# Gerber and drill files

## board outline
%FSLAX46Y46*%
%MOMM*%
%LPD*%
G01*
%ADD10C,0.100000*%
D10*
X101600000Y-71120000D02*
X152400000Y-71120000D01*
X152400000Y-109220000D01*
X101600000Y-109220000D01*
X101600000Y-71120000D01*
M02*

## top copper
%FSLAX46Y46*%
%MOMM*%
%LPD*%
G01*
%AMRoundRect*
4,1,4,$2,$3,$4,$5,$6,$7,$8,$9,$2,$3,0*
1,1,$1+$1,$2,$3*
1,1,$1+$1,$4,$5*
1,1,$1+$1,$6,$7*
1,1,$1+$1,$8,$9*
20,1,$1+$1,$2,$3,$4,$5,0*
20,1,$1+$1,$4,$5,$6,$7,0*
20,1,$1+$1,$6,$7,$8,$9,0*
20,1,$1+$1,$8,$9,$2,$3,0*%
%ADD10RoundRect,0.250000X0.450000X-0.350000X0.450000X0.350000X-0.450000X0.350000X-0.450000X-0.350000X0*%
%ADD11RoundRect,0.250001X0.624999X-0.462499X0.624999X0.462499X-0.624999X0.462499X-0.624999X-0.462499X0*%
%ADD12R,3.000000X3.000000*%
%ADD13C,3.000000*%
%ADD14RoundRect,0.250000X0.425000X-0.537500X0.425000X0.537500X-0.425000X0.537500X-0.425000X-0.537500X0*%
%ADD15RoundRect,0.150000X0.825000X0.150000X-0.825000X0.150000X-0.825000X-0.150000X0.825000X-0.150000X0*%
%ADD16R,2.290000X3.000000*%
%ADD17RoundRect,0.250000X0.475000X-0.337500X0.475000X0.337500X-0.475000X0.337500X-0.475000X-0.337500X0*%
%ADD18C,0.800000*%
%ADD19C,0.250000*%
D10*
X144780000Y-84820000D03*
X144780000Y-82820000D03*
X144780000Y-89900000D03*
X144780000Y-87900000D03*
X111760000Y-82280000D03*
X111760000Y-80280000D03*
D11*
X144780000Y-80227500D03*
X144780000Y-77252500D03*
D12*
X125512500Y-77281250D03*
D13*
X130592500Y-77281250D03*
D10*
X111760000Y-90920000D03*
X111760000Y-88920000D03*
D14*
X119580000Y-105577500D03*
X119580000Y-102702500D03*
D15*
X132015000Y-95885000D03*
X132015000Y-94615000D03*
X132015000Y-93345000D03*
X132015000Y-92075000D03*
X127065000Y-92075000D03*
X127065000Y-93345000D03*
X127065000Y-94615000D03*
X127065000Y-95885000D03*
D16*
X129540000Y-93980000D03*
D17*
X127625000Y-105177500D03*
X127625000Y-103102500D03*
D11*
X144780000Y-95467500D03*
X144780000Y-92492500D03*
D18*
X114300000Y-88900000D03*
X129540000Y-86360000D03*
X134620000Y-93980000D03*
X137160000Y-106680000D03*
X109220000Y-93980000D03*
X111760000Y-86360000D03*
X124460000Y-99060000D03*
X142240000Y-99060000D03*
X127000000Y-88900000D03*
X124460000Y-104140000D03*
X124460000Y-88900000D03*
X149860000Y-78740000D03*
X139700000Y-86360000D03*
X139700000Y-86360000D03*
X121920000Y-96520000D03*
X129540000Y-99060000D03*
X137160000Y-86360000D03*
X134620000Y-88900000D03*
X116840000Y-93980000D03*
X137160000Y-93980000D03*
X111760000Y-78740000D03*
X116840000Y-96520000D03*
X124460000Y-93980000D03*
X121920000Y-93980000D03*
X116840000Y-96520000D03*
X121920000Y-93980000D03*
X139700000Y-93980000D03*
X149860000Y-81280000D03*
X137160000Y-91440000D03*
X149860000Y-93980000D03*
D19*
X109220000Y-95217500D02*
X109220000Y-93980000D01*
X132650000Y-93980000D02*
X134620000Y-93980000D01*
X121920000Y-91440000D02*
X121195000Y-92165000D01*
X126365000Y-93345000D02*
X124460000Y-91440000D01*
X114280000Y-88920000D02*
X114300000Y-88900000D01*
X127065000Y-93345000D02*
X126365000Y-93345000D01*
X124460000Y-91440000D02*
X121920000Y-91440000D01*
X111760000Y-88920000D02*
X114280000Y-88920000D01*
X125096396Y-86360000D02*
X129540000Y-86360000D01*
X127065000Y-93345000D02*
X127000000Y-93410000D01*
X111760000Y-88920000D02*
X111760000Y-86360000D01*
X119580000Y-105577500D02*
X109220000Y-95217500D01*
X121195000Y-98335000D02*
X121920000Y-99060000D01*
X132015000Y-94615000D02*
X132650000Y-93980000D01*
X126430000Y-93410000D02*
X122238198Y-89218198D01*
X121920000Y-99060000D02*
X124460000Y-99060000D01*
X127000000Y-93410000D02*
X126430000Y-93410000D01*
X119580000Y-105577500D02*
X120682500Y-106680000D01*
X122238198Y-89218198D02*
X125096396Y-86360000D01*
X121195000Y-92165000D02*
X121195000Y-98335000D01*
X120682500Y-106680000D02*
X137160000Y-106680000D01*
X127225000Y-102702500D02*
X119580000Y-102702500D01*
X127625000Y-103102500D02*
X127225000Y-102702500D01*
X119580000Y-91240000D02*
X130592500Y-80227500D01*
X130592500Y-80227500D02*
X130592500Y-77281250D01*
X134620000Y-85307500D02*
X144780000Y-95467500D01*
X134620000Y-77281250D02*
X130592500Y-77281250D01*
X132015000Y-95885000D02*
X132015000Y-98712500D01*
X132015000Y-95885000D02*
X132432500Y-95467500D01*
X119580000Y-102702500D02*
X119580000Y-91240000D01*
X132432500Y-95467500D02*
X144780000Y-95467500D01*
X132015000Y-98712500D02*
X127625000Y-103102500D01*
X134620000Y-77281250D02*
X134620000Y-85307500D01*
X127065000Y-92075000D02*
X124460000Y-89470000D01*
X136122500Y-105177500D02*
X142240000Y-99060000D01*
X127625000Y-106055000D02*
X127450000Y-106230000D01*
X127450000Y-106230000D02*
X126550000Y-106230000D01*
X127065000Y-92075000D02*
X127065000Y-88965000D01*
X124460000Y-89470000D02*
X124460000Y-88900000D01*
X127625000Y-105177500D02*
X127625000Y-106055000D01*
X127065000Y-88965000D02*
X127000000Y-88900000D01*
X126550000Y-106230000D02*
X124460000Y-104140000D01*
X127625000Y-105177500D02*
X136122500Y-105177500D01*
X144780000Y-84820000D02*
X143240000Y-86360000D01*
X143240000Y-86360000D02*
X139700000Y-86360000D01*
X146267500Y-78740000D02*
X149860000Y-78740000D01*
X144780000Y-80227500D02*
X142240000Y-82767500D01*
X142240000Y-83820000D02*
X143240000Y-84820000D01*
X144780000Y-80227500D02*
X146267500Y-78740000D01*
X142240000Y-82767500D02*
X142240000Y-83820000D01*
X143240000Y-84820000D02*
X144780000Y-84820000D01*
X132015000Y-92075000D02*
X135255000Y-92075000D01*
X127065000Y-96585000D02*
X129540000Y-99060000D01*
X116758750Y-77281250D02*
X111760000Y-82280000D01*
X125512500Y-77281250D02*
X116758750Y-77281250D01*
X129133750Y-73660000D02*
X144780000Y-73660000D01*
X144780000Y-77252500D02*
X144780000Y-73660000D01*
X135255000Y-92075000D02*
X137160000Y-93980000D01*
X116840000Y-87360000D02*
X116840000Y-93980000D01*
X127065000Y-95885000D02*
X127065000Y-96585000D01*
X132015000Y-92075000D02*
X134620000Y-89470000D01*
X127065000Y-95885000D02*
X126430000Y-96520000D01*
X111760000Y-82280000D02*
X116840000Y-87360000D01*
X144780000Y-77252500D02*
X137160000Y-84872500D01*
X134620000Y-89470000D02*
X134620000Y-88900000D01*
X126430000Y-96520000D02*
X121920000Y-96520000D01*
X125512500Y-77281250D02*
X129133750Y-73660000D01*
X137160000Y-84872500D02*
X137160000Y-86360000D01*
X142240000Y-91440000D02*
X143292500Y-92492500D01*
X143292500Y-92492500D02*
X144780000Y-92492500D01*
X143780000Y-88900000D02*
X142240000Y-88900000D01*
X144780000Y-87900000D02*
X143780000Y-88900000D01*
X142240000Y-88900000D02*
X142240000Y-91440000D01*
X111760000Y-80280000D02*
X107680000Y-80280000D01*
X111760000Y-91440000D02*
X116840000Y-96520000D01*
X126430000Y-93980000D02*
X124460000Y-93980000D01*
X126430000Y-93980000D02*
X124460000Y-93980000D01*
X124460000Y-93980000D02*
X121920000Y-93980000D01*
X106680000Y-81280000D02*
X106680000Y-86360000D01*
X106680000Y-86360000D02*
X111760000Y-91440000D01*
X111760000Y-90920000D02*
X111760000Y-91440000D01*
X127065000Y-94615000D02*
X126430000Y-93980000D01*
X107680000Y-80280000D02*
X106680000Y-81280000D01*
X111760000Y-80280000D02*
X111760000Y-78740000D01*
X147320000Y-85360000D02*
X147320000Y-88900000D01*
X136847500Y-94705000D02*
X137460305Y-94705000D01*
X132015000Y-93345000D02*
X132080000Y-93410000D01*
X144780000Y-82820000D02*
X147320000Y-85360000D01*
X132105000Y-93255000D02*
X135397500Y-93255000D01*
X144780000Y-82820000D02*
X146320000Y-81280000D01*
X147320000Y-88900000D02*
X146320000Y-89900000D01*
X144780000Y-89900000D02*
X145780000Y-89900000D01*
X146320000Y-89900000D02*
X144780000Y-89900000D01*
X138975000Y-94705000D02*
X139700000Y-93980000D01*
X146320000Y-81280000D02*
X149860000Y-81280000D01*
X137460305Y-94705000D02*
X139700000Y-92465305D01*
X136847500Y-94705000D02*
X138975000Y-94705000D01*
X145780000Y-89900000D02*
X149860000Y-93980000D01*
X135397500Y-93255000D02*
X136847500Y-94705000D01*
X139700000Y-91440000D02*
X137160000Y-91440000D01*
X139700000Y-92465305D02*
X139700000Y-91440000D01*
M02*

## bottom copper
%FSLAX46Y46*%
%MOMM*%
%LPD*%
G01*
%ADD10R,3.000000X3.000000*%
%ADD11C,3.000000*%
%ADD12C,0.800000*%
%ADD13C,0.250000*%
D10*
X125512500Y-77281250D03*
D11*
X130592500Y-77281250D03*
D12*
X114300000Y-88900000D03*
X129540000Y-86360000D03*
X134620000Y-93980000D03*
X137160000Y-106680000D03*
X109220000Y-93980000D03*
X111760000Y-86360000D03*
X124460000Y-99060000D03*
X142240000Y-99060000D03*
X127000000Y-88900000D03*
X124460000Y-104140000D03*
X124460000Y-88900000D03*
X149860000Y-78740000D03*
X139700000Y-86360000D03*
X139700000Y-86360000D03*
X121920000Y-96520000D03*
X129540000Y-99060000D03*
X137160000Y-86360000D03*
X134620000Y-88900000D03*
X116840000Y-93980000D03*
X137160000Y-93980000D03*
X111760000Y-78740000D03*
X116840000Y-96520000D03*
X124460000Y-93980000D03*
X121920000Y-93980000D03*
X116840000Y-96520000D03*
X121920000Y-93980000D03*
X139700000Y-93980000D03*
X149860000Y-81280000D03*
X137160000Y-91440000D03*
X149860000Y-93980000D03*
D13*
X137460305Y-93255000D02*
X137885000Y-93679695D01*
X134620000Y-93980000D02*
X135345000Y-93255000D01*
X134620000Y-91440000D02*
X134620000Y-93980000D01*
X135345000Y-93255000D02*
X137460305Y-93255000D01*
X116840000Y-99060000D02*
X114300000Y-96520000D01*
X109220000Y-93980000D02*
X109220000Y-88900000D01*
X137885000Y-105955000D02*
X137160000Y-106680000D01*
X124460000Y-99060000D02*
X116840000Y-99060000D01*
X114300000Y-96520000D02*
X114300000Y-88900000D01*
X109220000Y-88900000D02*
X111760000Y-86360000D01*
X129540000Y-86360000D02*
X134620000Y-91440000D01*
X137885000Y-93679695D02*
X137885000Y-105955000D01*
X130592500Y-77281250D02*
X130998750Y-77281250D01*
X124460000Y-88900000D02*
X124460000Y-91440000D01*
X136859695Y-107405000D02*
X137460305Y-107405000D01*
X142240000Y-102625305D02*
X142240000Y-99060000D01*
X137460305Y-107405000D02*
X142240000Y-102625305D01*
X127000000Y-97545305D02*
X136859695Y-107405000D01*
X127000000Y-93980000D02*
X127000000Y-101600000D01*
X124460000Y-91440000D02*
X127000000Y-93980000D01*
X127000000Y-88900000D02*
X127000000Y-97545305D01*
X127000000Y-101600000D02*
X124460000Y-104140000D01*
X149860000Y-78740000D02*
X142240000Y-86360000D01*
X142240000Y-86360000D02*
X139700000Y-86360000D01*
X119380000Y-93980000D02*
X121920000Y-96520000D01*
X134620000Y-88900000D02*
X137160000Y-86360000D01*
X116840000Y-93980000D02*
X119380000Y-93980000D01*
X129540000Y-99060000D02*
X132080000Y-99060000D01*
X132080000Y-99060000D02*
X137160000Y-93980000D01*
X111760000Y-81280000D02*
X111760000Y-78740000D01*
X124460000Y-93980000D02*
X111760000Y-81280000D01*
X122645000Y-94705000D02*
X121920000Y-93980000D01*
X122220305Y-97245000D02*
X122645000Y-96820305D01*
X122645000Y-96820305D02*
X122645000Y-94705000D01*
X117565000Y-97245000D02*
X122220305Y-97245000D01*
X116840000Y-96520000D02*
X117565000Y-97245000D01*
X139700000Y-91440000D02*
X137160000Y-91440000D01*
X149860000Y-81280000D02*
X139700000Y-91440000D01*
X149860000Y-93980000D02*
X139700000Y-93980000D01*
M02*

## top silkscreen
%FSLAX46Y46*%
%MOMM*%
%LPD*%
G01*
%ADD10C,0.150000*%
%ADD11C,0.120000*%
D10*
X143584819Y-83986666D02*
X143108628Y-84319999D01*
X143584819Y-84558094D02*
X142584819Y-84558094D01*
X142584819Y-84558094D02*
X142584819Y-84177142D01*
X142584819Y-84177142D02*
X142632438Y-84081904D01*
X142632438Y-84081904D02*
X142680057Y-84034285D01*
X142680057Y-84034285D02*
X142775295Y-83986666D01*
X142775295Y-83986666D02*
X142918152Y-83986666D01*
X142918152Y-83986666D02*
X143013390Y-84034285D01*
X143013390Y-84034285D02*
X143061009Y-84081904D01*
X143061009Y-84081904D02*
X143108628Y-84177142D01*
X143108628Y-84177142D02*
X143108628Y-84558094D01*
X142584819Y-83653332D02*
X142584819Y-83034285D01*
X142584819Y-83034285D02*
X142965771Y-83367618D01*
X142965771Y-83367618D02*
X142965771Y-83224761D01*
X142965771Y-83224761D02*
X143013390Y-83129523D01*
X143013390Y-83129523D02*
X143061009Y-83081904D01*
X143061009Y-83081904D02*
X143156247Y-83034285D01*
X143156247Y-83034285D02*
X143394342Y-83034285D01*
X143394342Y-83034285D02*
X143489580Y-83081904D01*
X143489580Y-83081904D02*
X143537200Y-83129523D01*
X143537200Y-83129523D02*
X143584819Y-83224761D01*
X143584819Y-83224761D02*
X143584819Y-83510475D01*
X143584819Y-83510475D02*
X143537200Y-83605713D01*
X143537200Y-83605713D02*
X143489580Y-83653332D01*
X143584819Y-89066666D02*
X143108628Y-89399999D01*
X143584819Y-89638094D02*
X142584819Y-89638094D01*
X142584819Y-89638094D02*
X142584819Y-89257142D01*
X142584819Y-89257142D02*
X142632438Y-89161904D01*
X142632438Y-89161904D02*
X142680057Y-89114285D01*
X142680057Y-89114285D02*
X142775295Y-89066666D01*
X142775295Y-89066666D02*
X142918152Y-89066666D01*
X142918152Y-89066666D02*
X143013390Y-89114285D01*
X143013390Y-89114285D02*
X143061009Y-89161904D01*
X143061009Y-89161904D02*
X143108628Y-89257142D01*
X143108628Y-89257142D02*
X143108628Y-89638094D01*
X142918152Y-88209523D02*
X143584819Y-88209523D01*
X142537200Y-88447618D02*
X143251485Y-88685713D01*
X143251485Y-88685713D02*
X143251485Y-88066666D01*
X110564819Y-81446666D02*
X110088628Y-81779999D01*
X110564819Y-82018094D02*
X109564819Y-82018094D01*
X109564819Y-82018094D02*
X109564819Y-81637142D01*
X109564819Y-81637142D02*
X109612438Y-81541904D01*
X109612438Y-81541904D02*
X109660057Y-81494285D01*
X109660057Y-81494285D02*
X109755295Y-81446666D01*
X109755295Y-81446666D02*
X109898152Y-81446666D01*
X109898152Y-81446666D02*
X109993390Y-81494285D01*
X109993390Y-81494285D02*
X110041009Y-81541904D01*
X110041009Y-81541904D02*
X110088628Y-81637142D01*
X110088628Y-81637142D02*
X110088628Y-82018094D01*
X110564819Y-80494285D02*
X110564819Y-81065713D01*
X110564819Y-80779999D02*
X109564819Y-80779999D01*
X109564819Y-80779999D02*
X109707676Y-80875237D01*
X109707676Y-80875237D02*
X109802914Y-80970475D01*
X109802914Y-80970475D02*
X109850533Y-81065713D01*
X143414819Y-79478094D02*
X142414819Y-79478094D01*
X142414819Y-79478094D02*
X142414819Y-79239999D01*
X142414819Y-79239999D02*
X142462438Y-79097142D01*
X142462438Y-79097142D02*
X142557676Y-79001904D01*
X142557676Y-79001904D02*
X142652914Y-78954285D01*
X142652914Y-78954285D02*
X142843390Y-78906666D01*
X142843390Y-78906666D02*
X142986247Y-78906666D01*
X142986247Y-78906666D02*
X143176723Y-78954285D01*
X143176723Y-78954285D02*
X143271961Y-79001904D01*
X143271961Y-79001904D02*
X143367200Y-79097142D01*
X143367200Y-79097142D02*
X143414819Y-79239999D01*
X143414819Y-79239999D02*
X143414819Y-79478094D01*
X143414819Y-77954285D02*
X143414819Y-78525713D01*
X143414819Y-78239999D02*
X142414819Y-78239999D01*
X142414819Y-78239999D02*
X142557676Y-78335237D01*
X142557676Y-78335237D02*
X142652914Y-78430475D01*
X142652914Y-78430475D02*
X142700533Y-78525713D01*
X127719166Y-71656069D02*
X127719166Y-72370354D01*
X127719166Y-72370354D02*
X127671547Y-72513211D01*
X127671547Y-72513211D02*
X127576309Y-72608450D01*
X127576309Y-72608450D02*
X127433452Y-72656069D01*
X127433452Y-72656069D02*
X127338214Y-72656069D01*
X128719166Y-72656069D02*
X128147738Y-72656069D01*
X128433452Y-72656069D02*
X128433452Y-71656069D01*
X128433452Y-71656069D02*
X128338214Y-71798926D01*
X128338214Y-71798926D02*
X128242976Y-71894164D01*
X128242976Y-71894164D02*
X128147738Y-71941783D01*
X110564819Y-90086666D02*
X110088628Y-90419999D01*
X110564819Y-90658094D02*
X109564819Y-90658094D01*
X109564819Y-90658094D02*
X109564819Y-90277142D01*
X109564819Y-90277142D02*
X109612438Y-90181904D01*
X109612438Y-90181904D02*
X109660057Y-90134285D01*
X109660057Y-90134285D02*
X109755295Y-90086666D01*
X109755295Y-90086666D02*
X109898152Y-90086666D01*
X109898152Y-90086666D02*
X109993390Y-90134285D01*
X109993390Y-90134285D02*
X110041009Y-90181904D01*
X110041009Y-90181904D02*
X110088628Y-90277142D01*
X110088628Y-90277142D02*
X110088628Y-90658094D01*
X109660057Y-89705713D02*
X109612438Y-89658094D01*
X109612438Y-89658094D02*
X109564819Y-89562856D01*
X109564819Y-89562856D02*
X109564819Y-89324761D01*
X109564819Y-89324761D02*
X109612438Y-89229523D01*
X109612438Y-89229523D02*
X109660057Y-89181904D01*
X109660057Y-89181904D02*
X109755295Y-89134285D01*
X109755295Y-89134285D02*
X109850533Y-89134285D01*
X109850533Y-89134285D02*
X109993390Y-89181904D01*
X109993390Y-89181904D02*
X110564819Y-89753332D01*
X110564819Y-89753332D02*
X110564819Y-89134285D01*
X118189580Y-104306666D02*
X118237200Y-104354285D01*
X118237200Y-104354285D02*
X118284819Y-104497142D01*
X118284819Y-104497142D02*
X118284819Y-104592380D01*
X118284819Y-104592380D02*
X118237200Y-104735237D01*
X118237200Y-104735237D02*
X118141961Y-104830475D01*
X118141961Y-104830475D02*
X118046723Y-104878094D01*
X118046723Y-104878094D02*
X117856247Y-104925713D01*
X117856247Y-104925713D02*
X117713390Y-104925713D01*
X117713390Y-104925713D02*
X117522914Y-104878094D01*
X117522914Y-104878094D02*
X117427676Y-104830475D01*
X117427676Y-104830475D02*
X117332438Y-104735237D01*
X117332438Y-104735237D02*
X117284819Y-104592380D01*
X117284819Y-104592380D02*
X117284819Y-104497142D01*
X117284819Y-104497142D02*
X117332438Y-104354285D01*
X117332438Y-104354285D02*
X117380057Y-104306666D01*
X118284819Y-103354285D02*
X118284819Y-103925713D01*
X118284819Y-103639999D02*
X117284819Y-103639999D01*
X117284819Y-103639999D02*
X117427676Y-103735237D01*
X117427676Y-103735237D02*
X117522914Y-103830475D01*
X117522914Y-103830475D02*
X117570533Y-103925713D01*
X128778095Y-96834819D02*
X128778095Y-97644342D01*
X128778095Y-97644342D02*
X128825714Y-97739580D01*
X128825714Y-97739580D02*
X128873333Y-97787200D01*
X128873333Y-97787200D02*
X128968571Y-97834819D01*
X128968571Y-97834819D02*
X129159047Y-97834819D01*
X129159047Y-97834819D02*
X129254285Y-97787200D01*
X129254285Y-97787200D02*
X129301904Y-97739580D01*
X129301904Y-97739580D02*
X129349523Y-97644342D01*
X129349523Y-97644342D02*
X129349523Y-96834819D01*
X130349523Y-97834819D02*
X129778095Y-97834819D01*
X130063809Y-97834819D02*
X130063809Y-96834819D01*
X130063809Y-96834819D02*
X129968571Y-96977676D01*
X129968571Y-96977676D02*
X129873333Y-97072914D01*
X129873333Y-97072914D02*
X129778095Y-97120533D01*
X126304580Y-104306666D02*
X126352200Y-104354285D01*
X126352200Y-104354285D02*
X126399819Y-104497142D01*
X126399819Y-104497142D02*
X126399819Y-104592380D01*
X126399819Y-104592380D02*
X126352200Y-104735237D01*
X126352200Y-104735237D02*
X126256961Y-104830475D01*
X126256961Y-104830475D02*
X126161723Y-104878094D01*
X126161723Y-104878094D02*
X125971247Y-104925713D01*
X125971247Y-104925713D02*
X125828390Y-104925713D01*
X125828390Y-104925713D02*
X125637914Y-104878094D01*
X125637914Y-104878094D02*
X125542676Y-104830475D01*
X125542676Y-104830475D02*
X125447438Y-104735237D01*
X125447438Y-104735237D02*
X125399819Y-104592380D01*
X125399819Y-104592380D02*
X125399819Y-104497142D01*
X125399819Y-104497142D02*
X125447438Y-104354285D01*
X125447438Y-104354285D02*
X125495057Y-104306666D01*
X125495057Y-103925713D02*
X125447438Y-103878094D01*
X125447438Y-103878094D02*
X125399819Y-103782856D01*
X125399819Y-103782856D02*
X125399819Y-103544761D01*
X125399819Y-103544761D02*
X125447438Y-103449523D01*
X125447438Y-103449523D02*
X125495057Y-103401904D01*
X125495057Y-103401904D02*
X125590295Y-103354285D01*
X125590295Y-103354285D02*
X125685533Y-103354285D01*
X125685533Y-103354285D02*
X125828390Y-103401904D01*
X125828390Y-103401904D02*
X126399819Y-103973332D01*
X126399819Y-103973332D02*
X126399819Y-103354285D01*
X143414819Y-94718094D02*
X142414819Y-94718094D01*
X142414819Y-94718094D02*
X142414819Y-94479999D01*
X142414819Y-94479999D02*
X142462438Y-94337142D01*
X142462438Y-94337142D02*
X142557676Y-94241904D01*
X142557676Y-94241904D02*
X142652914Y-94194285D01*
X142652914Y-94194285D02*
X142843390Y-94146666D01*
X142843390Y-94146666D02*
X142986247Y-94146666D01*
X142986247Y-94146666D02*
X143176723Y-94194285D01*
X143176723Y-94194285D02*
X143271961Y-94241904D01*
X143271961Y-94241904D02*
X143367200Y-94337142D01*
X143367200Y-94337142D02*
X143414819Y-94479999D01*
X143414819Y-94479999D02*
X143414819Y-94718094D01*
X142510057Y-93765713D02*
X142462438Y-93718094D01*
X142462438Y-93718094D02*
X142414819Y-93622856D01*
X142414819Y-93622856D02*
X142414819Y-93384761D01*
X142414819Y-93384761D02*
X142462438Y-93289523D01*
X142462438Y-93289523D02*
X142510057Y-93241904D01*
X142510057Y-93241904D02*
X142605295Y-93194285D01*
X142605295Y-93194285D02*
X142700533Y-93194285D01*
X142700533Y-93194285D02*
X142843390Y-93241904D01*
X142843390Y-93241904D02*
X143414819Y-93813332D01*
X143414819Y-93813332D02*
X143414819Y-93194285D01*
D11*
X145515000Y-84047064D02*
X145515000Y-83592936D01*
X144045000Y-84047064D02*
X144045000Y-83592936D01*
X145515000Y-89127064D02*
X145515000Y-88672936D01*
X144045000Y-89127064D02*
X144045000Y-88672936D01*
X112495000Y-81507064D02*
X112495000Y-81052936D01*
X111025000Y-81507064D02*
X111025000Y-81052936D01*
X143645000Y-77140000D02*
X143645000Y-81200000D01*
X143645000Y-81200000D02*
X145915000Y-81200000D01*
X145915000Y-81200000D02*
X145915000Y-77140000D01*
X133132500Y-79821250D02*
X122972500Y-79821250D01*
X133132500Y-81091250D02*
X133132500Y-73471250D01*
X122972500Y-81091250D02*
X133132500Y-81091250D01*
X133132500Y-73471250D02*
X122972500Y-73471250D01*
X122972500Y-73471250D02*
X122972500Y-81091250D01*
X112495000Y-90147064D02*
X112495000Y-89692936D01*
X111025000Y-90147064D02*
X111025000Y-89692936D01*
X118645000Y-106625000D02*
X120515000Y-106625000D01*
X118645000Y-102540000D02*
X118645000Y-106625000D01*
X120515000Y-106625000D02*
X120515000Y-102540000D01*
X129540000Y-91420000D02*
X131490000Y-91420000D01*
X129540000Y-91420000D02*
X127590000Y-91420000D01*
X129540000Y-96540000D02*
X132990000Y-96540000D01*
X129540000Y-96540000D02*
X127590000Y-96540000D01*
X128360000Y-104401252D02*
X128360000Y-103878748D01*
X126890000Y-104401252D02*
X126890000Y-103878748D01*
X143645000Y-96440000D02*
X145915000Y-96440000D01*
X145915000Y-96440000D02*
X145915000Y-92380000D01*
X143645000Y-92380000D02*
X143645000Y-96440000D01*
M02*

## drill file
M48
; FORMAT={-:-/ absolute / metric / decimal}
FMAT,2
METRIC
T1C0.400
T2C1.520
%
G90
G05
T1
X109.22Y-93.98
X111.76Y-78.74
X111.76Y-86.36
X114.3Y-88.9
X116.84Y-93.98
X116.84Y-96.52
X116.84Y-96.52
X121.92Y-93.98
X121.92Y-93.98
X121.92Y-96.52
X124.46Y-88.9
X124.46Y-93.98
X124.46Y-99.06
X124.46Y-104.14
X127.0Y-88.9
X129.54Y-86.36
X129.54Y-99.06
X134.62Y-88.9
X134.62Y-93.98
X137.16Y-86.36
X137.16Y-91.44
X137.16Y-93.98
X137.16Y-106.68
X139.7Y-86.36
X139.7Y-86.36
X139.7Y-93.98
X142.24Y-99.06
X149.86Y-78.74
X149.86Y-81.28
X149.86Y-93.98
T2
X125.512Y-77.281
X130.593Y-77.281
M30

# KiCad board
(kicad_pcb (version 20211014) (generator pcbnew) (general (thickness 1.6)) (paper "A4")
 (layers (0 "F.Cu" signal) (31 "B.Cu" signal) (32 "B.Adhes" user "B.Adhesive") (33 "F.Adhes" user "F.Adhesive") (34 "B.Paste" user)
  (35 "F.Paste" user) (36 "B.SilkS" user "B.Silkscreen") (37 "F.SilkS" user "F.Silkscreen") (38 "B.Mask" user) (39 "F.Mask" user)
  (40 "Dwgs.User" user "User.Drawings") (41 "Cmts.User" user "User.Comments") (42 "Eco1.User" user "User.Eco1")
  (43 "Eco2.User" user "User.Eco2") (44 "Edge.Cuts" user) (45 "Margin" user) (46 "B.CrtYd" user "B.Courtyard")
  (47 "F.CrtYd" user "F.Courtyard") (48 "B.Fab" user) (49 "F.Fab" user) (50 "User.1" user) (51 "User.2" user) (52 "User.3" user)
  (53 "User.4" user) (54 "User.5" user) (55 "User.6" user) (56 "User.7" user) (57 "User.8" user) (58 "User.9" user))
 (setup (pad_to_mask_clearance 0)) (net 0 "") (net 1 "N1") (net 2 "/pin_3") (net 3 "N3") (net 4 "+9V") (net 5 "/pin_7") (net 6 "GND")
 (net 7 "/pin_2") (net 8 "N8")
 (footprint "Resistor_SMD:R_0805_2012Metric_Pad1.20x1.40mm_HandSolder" (layer "F.Cu") (at 144.78 83.82 90)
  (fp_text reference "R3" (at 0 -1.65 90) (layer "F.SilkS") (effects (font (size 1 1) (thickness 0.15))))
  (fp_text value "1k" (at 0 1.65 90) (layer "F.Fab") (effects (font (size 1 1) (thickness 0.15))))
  (fp_line (start -0.227064 0.735) (end 0.227064 0.735) (layer "F.SilkS") (width 0.12))
  (fp_line (start -0.227064 -0.735) (end 0.227064 -0.735) (layer "F.SilkS") (width 0.12))
  (pad "1" smd roundrect (at -1 0 90) (size 1.2 1.4) (layers "F.Cu" "F.Paste" "F.Mask") (roundrect_rratio 0.208333) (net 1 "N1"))
  (pad "2" smd roundrect (at 1 0 90) (size 1.2 1.4) (layers "F.Cu" "F.Paste" "F.Mask") (roundrect_rratio 0.208333) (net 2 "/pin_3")))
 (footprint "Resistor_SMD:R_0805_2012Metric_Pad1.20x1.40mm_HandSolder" (layer "F.Cu") (at 144.78 88.9 90)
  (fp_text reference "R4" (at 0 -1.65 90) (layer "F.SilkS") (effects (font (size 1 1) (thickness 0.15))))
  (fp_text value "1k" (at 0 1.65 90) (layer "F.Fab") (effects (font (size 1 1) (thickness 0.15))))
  (fp_line (start -0.227064 0.735) (end 0.227064 0.735) (layer "F.SilkS") (width 0.12))
  (fp_line (start -0.227064 -0.735) (end 0.227064 -0.735) (layer "F.SilkS") (width 0.12))
  (pad "1" smd roundrect (at -1 0 90) (size 1.2 1.4) (layers "F.Cu" "F.Paste" "F.Mask") (roundrect_rratio 0.208333) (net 2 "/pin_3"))
  (pad "2" smd roundrect (at 1 0 90) (size 1.2 1.4) (layers "F.Cu" "F.Paste" "F.Mask") (roundrect_rratio 0.208333) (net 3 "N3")))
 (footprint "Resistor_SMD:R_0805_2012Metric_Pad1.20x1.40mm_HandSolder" (layer "F.Cu") (at 111.76 81.28 90)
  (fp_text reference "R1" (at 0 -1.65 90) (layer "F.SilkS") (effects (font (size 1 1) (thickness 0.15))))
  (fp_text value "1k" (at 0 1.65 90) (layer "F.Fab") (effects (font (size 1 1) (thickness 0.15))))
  (fp_line (start -0.227064 0.735) (end 0.227064 0.735) (layer "F.SilkS") (width 0.12))
  (fp_line (start -0.227064 -0.735) (end 0.227064 -0.735) (layer "F.SilkS") (width 0.12))
  (pad "1" smd roundrect (at -1 0 90) (size 1.2 1.4) (layers "F.Cu" "F.Paste" "F.Mask") (roundrect_rratio 0.208333) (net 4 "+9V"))
  (pad "2" smd roundrect (at 1 0 90) (size 1.2 1.4) (layers "F.Cu" "F.Paste" "F.Mask") (roundrect_rratio 0.208333) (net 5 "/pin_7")))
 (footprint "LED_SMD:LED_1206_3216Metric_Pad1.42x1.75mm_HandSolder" (layer "F.Cu") (at 144.78 78.74 90)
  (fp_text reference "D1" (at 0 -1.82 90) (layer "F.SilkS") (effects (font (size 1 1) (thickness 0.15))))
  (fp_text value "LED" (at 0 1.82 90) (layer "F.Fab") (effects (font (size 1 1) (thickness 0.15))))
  (fp_line (start 1.6 -1.135) (end -2.46 -1.135) (layer "F.SilkS") (width 0.12))
  (fp_line (start -2.46 -1.135) (end -2.46 1.135) (layer "F.SilkS") (width 0.12))
  (fp_line (start -2.46 1.135) (end 1.6 1.135) (layer "F.SilkS") (width 0.12))
  (pad "1" smd roundrect (at -1.4875 0 90) (size 1.425 1.75) (layers "F.Cu" "F.Paste" "F.Mask") (roundrect_rratio 0.175439) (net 1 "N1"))
  (pad "2" smd roundrect (at 1.4875 0 90) (size 1.425 1.75) (layers "F.Cu" "F.Paste" "F.Mask") (roundrect_rratio 0.175439) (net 4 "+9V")))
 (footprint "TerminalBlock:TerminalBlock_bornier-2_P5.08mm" (layer "F.Cu") (at 125.5125 77.28125)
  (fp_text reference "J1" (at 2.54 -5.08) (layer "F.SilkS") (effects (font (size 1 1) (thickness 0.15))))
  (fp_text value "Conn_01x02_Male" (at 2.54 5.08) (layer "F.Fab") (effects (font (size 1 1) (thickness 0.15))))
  (fp_line (start 7.62 2.54) (end -2.54 2.54) (layer "F.SilkS") (width 0.12))
  (fp_line (start 7.62 3.81) (end 7.62 -3.81) (layer "F.SilkS") (width 0.12))
  (fp_line (start -2.54 3.81) (end 7.62 3.81) (layer "F.SilkS") (width 0.12))
  (fp_line (start 7.62 -3.81) (end -2.54 -3.81) (layer "F.SilkS") (width 0.12))
  (fp_line (start -2.54 -3.81) (end -2.54 3.81) (layer "F.SilkS") (width 0.12))
  (pad "1" thru_hole rect (at 0 0) (size 3 3) (drill 1.52) (layers *.Cu *.Mask) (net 4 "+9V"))
  (pad "2" thru_hole circle (at 5.08 0) (size 3 3) (drill 1.52) (layers *.Cu *.Mask) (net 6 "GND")))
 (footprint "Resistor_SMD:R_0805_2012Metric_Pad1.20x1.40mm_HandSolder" (layer "F.Cu") (at 111.76 89.92 90)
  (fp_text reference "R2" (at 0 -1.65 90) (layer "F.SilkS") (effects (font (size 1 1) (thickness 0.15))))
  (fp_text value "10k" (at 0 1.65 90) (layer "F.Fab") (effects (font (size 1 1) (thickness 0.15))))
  (fp_line (start -0.227064 0.735) (end 0.227064 0.735) (layer "F.SilkS") (width 0.12))
  (fp_line (start -0.227064 -0.735) (end 0.227064 -0.735) (layer "F.SilkS") (width 0.12))
  (pad "1" smd roundrect (at -1 0 90) (size 1.2 1.4) (layers "F.Cu" "F.Paste" "F.Mask") (roundrect_rratio 0.208333) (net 5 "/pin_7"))
  (pad "2" smd roundrect (at 1 0 90) (size 1.2 1.4) (layers "F.Cu" "F.Paste" "F.Mask") (roundrect_rratio 0.208333) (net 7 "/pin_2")))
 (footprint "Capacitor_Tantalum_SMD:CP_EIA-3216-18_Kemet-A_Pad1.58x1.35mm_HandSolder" (layer "F.Cu") (at 119.58 104.14 90)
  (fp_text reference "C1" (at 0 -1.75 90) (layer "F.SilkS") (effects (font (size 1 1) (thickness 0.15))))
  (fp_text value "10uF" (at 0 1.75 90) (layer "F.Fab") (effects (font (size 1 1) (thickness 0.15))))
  (fp_line (start -2.485 -0.935) (end -2.485 0.935) (layer "F.SilkS") (width 0.12))
  (fp_line (start 1.6 -0.935) (end -2.485 -0.935) (layer "F.SilkS") (width 0.12))
  (fp_line (start -2.485 0.935) (end 1.6 0.935) (layer "F.SilkS") (width 0.12))
  (pad "1" smd roundrect (at -1.4375 0 90) (size 1.575 1.35) (layers "F.Cu" "F.Paste" "F.Mask") (roundrect_rratio 0.185185) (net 7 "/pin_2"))
  (pad "2" smd roundrect (at 1.4375 0 90) (size 1.575 1.35) (layers "F.Cu" "F.Paste" "F.Mask") (roundrect_rratio 0.185185) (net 6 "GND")))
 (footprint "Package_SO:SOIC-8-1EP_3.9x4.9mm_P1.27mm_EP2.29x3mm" (layer "F.Cu") (at 129.54 93.98 180)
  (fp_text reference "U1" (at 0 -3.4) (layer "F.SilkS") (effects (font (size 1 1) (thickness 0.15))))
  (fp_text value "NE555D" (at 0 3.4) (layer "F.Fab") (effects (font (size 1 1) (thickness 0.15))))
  (fp_line (start 0 2.56) (end -1.95 2.56) (layer "F.SilkS") (width 0.12))
  (fp_line (start 0 2.56) (end 1.95 2.56) (layer "F.SilkS") (width 0.12))
  (fp_line (start 0 -2.56) (end -3.45 -2.56) (layer "F.SilkS") (width 0.12))
  (fp_line (start 0 -2.56) (end 1.95 -2.56) (layer "F.SilkS") (width 0.12))
  (pad "" smd roundrect (at -0.57 0.75 180) (size 0.92 1.21) (layers "F.Paste") (roundrect_rratio 0.25))
  (pad "" smd roundrect (at 0.57 -0.75 180) (size 0.92 1.21) (layers "F.Paste") (roundrect_rratio 0.25))
  (pad "" smd roundrect (at -0.57 -0.75 180) (size 0.92 1.21) (layers "F.Paste") (roundrect_rratio 0.25))
  (pad "" smd roundrect (at 0.57 0.75 180) (size 0.92 1.21) (layers "F.Paste") (roundrect_rratio 0.25))
  (pad "1" smd roundrect (at -2.475 -1.905 180) (size 1.95 0.6) (layers "F.Cu" "F.Paste" "F.Mask") (roundrect_rratio 0.25) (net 6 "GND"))
  (pad "2" smd roundrect (at -2.475 -0.635 180) (size 1.95 0.6) (layers "F.Cu" "F.Paste" "F.Mask") (roundrect_rratio 0.25) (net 7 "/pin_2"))
  (pad "3" smd roundrect (at -2.475 0.635 180) (size 1.95 0.6) (layers "F.Cu" "F.Paste" "F.Mask") (roundrect_rratio 0.25) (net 2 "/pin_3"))
  (pad "4" smd roundrect (at -2.475 1.905 180) (size 1.95 0.6) (layers "F.Cu" "F.Paste" "F.Mask") (roundrect_rratio 0.25) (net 4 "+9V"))
  (pad "5" smd roundrect (at 2.475 1.905 180) (size 1.95 0.6) (layers "F.Cu" "F.Paste" "F.Mask") (roundrect_rratio 0.25) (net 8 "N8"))
  (pad "6" smd roundrect (at 2.475 0.635 180) (size 1.95 0.6) (layers "F.Cu" "F.Paste" "F.Mask") (roundrect_rratio 0.25) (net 7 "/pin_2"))
  (pad "7" smd roundrect (at 2.475 -0.635 180) (size 1.95 0.6) (layers "F.Cu" "F.Paste" "F.Mask") (roundrect_rratio 0.25) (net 5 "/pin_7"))
  (pad "8" smd roundrect (at 2.475 -1.905 180) (size 1.95 0.6) (layers "F.Cu" "F.Paste" "F.Mask") (roundrect_rratio 0.25) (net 4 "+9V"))
  (pad "9" smd rect (at 0 0 180) (size 2.29 3) (layers "F.Cu" "F.Mask")))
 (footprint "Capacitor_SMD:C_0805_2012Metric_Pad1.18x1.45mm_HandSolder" (layer "F.Cu") (at 127.625 104.14 90)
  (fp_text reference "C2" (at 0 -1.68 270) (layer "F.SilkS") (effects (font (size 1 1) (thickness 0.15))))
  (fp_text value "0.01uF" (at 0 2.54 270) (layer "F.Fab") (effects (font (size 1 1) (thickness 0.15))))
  (fp_line (start -0.261252 0.735) (end 0.261252 0.735) (layer "F.SilkS") (width 0.12))
  (fp_line (start -0.261252 -0.735) (end 0.261252 -0.735) (layer "F.SilkS") (width 0.12))
  (pad "1" smd roundrect (at -1.0375 0 90) (size 1.175 1.45) (layers "F.Cu" "F.Paste" "F.Mask") (roundrect_rratio 0.212766) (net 8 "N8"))
  (pad "2" smd roundrect (at 1.0375 0 90) (size 1.175 1.45) (layers "F.Cu" "F.Paste" "F.Mask") (roundrect_rratio 0.212766) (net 6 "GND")))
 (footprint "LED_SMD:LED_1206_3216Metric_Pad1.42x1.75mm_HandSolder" (layer "F.Cu") (at 144.78 93.98 90)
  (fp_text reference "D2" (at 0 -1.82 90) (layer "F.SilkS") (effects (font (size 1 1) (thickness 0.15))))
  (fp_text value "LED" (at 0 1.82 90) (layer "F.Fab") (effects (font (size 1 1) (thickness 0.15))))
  (fp_line (start -2.46 -1.135) (end -2.46 1.135) (layer "F.SilkS") (width 0.12))
  (fp_line (start -2.46 1.135) (end 1.6 1.135) (layer "F.SilkS") (width 0.12))
  (fp_line (start 1.6 -1.135) (end -2.46 -1.135) (layer "F.SilkS") (width 0.12))
  (pad "1" smd roundrect (at -1.4875 0 90) (size 1.425 1.75) (layers "F.Cu" "F.Paste" "F.Mask") (roundrect_rratio 0.175439) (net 6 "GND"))
  (pad "2" smd roundrect (at 1.4875 0 90) (size 1.425 1.75) (layers "F.Cu" "F.Paste" "F.Mask") (roundrect_rratio 0.175439) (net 3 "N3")))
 (gr_rect (start 101.6 71.12) (end 152.4 109.22) (layer "Edge.Cuts") (width 0.1) (fill none))
 (segment (start 109.22 95.2175) (end 109.22 93.98) (width 0.25) (layer "F.Cu") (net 7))
 (segment (start 132.65 93.98) (end 134.62 93.98) (width 0.25) (layer "F.Cu") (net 7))
 (segment (start 121.92 91.44) (end 121.195 92.165) (width 0.25) (layer "F.Cu") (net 7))
 (segment (start 126.365 93.345) (end 124.46 91.44) (width 0.25) (layer "F.Cu") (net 7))
 (segment (start 114.28 88.92) (end 114.3 88.9) (width 0.25) (layer "F.Cu") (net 7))
 (segment (start 127.065 93.345) (end 126.365 93.345) (width 0.25) (layer "F.Cu") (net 7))
 (segment (start 124.46 91.44) (end 121.92 91.44) (width 0.25) (layer "F.Cu") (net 7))
 (segment (start 111.76 88.92) (end 114.28 88.92) (width 0.25) (layer "F.Cu") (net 7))
 (segment (start 125.096396 86.36) (end 129.54 86.36) (width 0.25) (layer "F.Cu") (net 7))
 (segment (start 127.065 93.345) (end 127 93.41) (width 0.25) (layer "F.Cu") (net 7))
 (segment (start 111.76 88.92) (end 111.76 86.36) (width 0.25) (layer "F.Cu") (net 7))
 (segment (start 119.58 105.5775) (end 109.22 95.2175) (width 0.25) (layer "F.Cu") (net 7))
 (segment (start 121.195 98.335) (end 121.92 99.06) (width 0.25) (layer "F.Cu") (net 7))
 (segment (start 132.015 94.615) (end 132.65 93.98) (width 0.25) (layer "F.Cu") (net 7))
 (segment (start 126.43 93.41) (end 122.238198 89.218198) (width 0.25) (layer "F.Cu") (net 7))
 (segment (start 121.92 99.06) (end 124.46 99.06) (width 0.25) (layer "F.Cu") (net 7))
 (segment (start 127 93.41) (end 126.43 93.41) (width 0.25) (layer "F.Cu") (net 7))
 (segment (start 119.58 105.5775) (end 120.6825 106.68) (width 0.25) (layer "F.Cu") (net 7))
 (segment (start 122.238198 89.218198) (end 125.096396 86.36) (width 0.25) (layer "F.Cu") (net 7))
 (segment (start 121.195 92.165) (end 121.195 98.335) (width 0.25) (layer "F.Cu") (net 7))
 (segment (start 120.6825 106.68) (end 137.16 106.68) (width 0.25) (layer "F.Cu") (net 7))
 (via (at 114.3 88.9) (size 0.8) (drill 0.4) (layers "F.Cu" "B.Cu") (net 7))
 (via (at 129.54 86.36) (size 0.8) (drill 0.4) (layers "F.Cu" "B.Cu") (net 7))
 (via (at 134.62 93.98) (size 0.8) (drill 0.4) (layers "F.Cu" "B.Cu") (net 7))
 (via (at 137.16 106.68) (size 0.8) (drill 0.4) (layers "F.Cu" "B.Cu") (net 7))
 (via (at 109.22 93.98) (size 0.8) (drill 0.4) (layers "F.Cu" "B.Cu") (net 7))
 (via (at 111.76 86.36) (size 0.8) (drill 0.4) (layers "F.Cu" "B.Cu") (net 7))
 (via (at 124.46 99.06) (size 0.8) (drill 0.4) (layers "F.Cu" "B.Cu") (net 7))
 (segment (start 137.460305 93.255) (end 137.885 93.679695) (width 0.25) (layer "B.Cu") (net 7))
 (segment (start 134.62 93.98) (end 135.345 93.255) (width 0.25) (layer "B.Cu") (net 7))
 (segment (start 134.62 91.44) (end 134.62 93.98) (width 0.25) (layer "B.Cu") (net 7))
 (segment (start 135.345 93.255) (end 137.460305 93.255) (width 0.25) (layer "B.Cu") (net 7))
 (segment (start 116.84 99.06) (end 114.3 96.52) (width 0.25) (layer "B.Cu") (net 7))
 (segment (start 109.22 93.98) (end 109.22 88.9) (width 0.25) (layer "B.Cu") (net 7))
 (segment (start 137.885 105.955) (end 137.16 106.68) (width 0.25) (layer "B.Cu") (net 7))
 (segment (start 124.46 99.06) (end 116.84 99.06) (width 0.25) (layer "B.Cu") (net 7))
 (segment (start 114.3 96.52) (end 114.3 88.9) (width 0.25) (layer "B.Cu") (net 7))
 (segment (start 109.22 88.9) (end 111.76 86.36) (width 0.25) (layer "B.Cu") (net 7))
 (segment (start 129.54 86.36) (end 134.62 91.44) (width 0.25) (layer "B.Cu") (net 7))
 (segment (start 137.885 93.679695) (end 137.885 105.955) (width 0.25) (layer "B.Cu") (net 7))
 (segment (start 127.225 102.7025) (end 119.58 102.7025) (width 0.25) (layer "F.Cu") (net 6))
 (segment (start 127.625 103.1025) (end 127.225 102.7025) (width 0.25) (layer "F.Cu") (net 6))
 (segment (start 119.58 91.24) (end 130.5925 80.2275) (width 0.25) (layer "F.Cu") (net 6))
 (segment (start 130.5925 80.2275) (end 130.5925 77.28125) (width 0.25) (layer "F.Cu") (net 6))
 (segment (start 134.62 85.3075) (end 144.78 95.4675) (width 0.25) (layer "F.Cu") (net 6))
 (segment (start 134.62 77.28125) (end 130.5925 77.28125) (width 0.25) (layer "F.Cu") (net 6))
 (segment (start 132.015 95.885) (end 132.015 98.7125) (width 0.25) (layer "F.Cu") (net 6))
 (segment (start 132.015 95.885) (end 132.4325 95.4675) (width 0.25) (layer "F.Cu") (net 6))
 (segment (start 119.58 102.7025) (end 119.58 91.24) (width 0.25) (layer "F.Cu") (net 6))
 (segment (start 132.4325 95.4675) (end 144.78 95.4675) (width 0.25) (layer "F.Cu") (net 6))
 (segment (start 132.015 98.7125) (end 127.625 103.1025) (width 0.25) (layer "F.Cu") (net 6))
 (segment (start 134.62 77.28125) (end 134.62 85.3075) (width 0.25) (layer "F.Cu") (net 6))
 (segment (start 130.5925 77.28125) (end 130.99875 77.28125) (width 0.25) (layer "B.Cu") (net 6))
 (segment (start 127.065 92.075) (end 124.46 89.47) (width 0.25) (layer "F.Cu") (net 8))
 (segment (start 136.1225 105.1775) (end 142.24 99.06) (width 0.25) (layer "F.Cu") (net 8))
 (segment (start 127.625 106.055) (end 127.45 106.23) (width 0.25) (layer "F.Cu") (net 8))
 (segment (start 127.45 106.23) (end 126.55 106.23) (width 0.25) (layer "F.Cu") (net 8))
 (segment (start 127.065 92.075) (end 127.065 88.965) (width 0.25) (layer "F.Cu") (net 8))
 (segment (start 124.46 89.47) (end 124.46 88.9) (width 0.25) (layer "F.Cu") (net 8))
 (segment (start 127.625 105.1775) (end 127.625 106.055) (width 0.25) (layer "F.Cu") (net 8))
 (segment (start 127.065 88.965) (end 127 88.9) (width 0.25) (layer "F.Cu") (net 8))
 (segment (start 126.55 106.23) (end 124.46 104.14) (width 0.25) (layer "F.Cu") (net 8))
 (segment (start 127.625 105.1775) (end 136.1225 105.1775) (width 0.25) (layer "F.Cu") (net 8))
 (via (at 142.24 99.06) (size 0.8) (drill 0.4) (layers "F.Cu" "B.Cu") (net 8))
 (via (at 127 88.9) (size 0.8) (drill 0.4) (layers "F.Cu" "B.Cu") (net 8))
 (via (at 124.46 104.14) (size 0.8) (drill 0.4) (layers "F.Cu" "B.Cu") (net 8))
 (via (at 124.46 88.9) (size 0.8) (drill 0.4) (layers "F.Cu" "B.Cu") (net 8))
 (segment (start 124.46 88.9) (end 124.46 91.44) (width 0.25) (layer "B.Cu") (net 8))
 (segment (start 136.859695 107.405) (end 137.460305 107.405) (width 0.25) (layer "B.Cu") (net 8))
 (segment (start 142.24 102.625305) (end 142.24 99.06) (width 0.25) (layer "B.Cu") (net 8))
 (segment (start 137.460305 107.405) (end 142.24 102.625305) (width 0.25) (layer "B.Cu") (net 8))
 (segment (start 127 97.545305) (end 136.859695 107.405) (width 0.25) (layer "B.Cu") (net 8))
 (segment (start 127 93.98) (end 127 101.6) (width 0.25) (layer "B.Cu") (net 8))
 (segment (start 124.46 91.44) (end 127 93.98) (width 0.25) (layer "B.Cu") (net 8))
 (segment (start 127 88.9) (end 127 97.545305) (width 0.25) (layer "B.Cu") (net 8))
 (segment (start 127 101.6) (end 124.46 104.14) (width 0.25) (layer "B.Cu") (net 8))
 (segment (start 144.78 84.82) (end 143.24 86.36) (width 0.25) (layer "F.Cu") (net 1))
 (segment (start 143.24 86.36) (end 139.7 86.36) (width 0.25) (layer "F.Cu") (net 1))
 (segment (start 146.2675 78.74) (end 149.86 78.74) (width 0.25) (layer "F.Cu") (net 1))
 (segment (start 144.78 80.2275) (end 142.24 82.7675) (width 0.25) (layer "F.Cu") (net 1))
 (segment (start 142.24 83.82) (end 143.24 84.82) (width 0.25) (layer "F.Cu") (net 1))
 (segment (start 144.78 80.2275) (end 146.2675 78.74) (width 0.25) (layer "F.Cu") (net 1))
 (segment (start 142.24 82.7675) (end 142.24 83.82) (width 0.25) (layer "F.Cu") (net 1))
 (segment (start 143.24 84.82) (end 144.78 84.82) (width 0.25) (layer "F.Cu") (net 1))
 (via (at 149.86 78.74) (size 0.8) (drill 0.4) (layers "F.Cu" "B.Cu") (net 1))
 (via (at 139.7 86.36) (size 0.8) (drill 0.4) (layers "F.Cu" "B.Cu") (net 1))
 (via (at 139.7 86.36) (size 0.8) (drill 0.4) (layers "F.Cu" "B.Cu") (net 1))
 (segment (start 149.86 78.74) (end 142.24 86.36) (width 0.25) (layer "B.Cu") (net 1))
 (segment (start 142.24 86.36) (end 139.7 86.36) (width 0.25) (layer "B.Cu") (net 1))
 (segment (start 132.015 92.075) (end 135.255 92.075) (width 0.25) (layer "F.Cu") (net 4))
 (segment (start 127.065 96.585) (end 129.54 99.06) (width 0.25) (layer "F.Cu") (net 4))
 (segment (start 116.75875 77.28125) (end 111.76 82.28) (width 0.25) (layer "F.Cu") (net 4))
 (segment (start 125.5125 77.28125) (end 116.75875 77.28125) (width 0.25) (layer "F.Cu") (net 4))
 (segment (start 129.13375 73.66) (end 144.78 73.66) (width 0.25) (layer "F.Cu") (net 4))
 (segment (start 144.78 77.2525) (end 144.78 73.66) (width 0.25) (layer "F.Cu") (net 4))
 (segment (start 135.255 92.075) (end 137.16 93.98) (width 0.25) (layer "F.Cu") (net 4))
 (segment (start 116.84 87.36) (end 116.84 93.98) (width 0.25) (layer "F.Cu") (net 4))
 (segment (start 127.065 95.885) (end 127.065 96.585) (width 0.25) (layer "F.Cu") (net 4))
 (segment (start 132.015 92.075) (end 134.62 89.47) (width 0.25) (layer "F.Cu") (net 4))
 (segment (start 127.065 95.885) (end 126.43 96.52) (width 0.25) (layer "F.Cu") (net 4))
 (segment (start 111.76 82.28) (end 116.84 87.36) (width 0.25) (layer "F.Cu") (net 4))
 (segment (start 144.78 77.2525) (end 137.16 84.8725) (width 0.25) (layer "F.Cu") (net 4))
 (segment (start 134.62 89.47) (end 134.62 88.9) (width 0.25) (layer "F.Cu") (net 4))
 (segment (start 126.43 96.52) (end 121.92 96.52) (width 0.25) (layer "F.Cu") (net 4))
 (segment (start 125.5125 77.28125) (end 129.13375 73.66) (width 0.25) (layer "F.Cu") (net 4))
 (segment (start 137.16 84.8725) (end 137.16 86.36) (width 0.25) (layer "F.Cu") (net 4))
 (via (at 121.92 96.52) (size 0.8) (drill 0.4) (layers "F.Cu" "B.Cu") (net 4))
 (via (at 129.54 99.06) (size 0.8) (drill 0.4) (layers "F.Cu" "B.Cu") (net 4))
 (via (at 137.16 86.36) (size 0.8) (drill 0.4) (layers "F.Cu" "B.Cu") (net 4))
 (via (at 134.62 88.9) (size 0.8) (drill 0.4) (layers "F.Cu" "B.Cu") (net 4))
 (via (at 116.84 93.98) (size 0.8) (drill 0.4) (layers "F.Cu" "B.Cu") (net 4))
 (via (at 137.16 93.98) (size 0.8) (drill 0.4) (layers "F.Cu" "B.Cu") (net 4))
 (segment (start 119.38 93.98) (end 121.92 96.52) (width 0.25) (layer "B.Cu") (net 4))
 (segment (start 134.62 88.9) (end 137.16 86.36) (width 0.25) (layer "B.Cu") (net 4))
 (segment (start 116.84 93.98) (end 119.38 93.98) (width 0.25) (layer "B.Cu") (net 4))
 (segment (start 129.54 99.06) (end 132.08 99.06) (width 0.25) (layer "B.Cu") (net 4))
 (segment (start 132.08 99.06) (end 137.16 93.98) (width 0.25) (layer "B.Cu") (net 4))
 (segment (start 142.24 91.44) (end 143.2925 92.4925) (width 0.25) (layer "F.Cu") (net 3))
 (segment (start 143.2925 92.4925) (end 144.78 92.4925) (width 0.25) (layer "F.Cu") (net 3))
 (segment (start 143.78 88.9) (end 142.24 88.9) (width 0.25) (layer "F.Cu") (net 3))
 (segment (start 144.78 87.9) (end 143.78 88.9) (width 0.25) (layer "F.Cu") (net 3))
 (segment (start 142.24 88.9) (end 142.24 91.44) (width 0.25) (layer "F.Cu") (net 3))
 (segment (start 111.76 80.28) (end 107.68 80.28) (width 0.25) (layer "F.Cu") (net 5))
 (segment (start 111.76 91.44) (end 116.84 96.52) (width 0.25) (layer "F.Cu") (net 5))
 (segment (start 126.43 93.98) (end 124.46 93.98) (width 0.25) (layer "F.Cu") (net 5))
 (segment (start 126.43 93.98) (end 124.46 93.98) (width 0.25) (layer "F.Cu") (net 5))
 (segment (start 124.46 93.98) (end 121.92 93.98) (width 0.25) (layer "F.Cu") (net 5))
 (segment (start 106.68 81.28) (end 106.68 86.36) (width 0.25) (layer "F.Cu") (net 5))
 (segment (start 106.68 86.36) (end 111.76 91.44) (width 0.25) (layer "F.Cu") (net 5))
 (segment (start 111.76 90.92) (end 111.76 91.44) (width 0.25) (layer "F.Cu") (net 5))
 (segment (start 127.065 94.615) (end 126.43 93.98) (width 0.25) (layer "F.Cu") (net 5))
 (segment (start 107.68 80.28) (end 106.68 81.28) (width 0.25) (layer "F.Cu") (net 5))
 (segment (start 111.76 80.28) (end 111.76 78.74) (width 0.25) (layer "F.Cu") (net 5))
 (via (at 111.76 78.74) (size 0.8) (drill 0.4) (layers "F.Cu" "B.Cu") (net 5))
 (via (at 116.84 96.52) (size 0.8) (drill 0.4) (layers "F.Cu" "B.Cu") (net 5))
 (via (at 124.46 93.98) (size 0.8) (drill 0.4) (layers "F.Cu" "B.Cu") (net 5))
 (via (at 121.92 93.98) (size 0.8) (drill 0.4) (layers "F.Cu" "B.Cu") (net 5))
 (via (at 116.84 96.52) (size 0.8) (drill 0.4) (layers "F.Cu" "B.Cu") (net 5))
 (via (at 121.92 93.98) (size 0.8) (drill 0.4) (layers "F.Cu" "B.Cu") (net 5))
 (segment (start 111.76 81.28) (end 111.76 78.74) (width 0.25) (layer "B.Cu") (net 5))
 (segment (start 124.46 93.98) (end 111.76 81.28) (width 0.25) (layer "B.Cu") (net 5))
 (segment (start 122.645 94.705) (end 121.92 93.98) (width 0.25) (layer "B.Cu") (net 5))
 (segment (start 122.220305 97.245) (end 122.645 96.820305) (width 0.25) (layer "B.Cu") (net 5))
 (segment (start 122.645 96.820305) (end 122.645 94.705) (width 0.25) (layer "B.Cu") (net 5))
 (segment (start 117.565 97.245) (end 122.220305 97.245) (width 0.25) (layer "B.Cu") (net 5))
 (segment (start 116.84 96.52) (end 117.565 97.245) (width 0.25) (layer "B.Cu") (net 5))
 (segment (start 147.32 85.36) (end 147.32 88.9) (width 0.25) (layer "F.Cu") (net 2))
 (segment (start 136.8475 94.705) (end 137.460305 94.705) (width 0.25) (layer "F.Cu") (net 2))
 (segment (start 132.015 93.345) (end 132.08 93.41) (width 0.25) (layer "F.Cu") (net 2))
 (segment (start 144.78 82.82) (end 147.32 85.36) (width 0.25) (layer "F.Cu") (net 2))
 (segment (start 132.105 93.255) (end 135.3975 93.255) (width 0.25) (layer "F.Cu") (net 2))
 (segment (start 144.78 82.82) (end 146.32 81.28) (width 0.25) (layer "F.Cu") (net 2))
 (segment (start 147.32 88.9) (end 146.32 89.9) (width 0.25) (layer "F.Cu") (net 2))
 (segment (start 144.78 89.9) (end 145.78 89.9) (width 0.25) (layer "F.Cu") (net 2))
 (segment (start 146.32 89.9) (end 144.78 89.9) (width 0.25) (layer "F.Cu") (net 2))
 (segment (start 138.975 94.705) (end 139.7 93.98) (width 0.25) (layer "F.Cu") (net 2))
 (segment (start 146.32 81.28) (end 149.86 81.28) (width 0.25) (layer "F.Cu") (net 2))
 (segment (start 137.460305 94.705) (end 139.7 92.465305) (width 0.25) (layer "F.Cu") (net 2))
 (segment (start 136.8475 94.705) (end 138.975 94.705) (width 0.25) (layer "F.Cu") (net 2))
 (segment (start 145.78 89.9) (end 149.86 93.98) (width 0.25) (layer "F.Cu") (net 2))
 (segment (start 135.3975 93.255) (end 136.8475 94.705) (width 0.25) (layer "F.Cu") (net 2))
 (segment (start 139.7 91.44) (end 137.16 91.44) (width 0.25) (layer "F.Cu") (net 2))
 (segment (start 139.7 92.465305) (end 139.7 91.44) (width 0.25) (layer "F.Cu") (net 2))
 (via (at 139.7 93.98) (size 0.8) (drill 0.4) (layers "F.Cu" "B.Cu") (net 2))
 (via (at 149.86 81.28) (size 0.8) (drill 0.4) (layers "F.Cu" "B.Cu") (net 2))
 (via (at 137.16 91.44) (size 0.8) (drill 0.4) (layers "F.Cu" "B.Cu") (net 2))
 (via (at 149.86 93.98) (size 0.8) (drill 0.4) (layers "F.Cu" "B.Cu") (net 2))
 (segment (start 139.7 91.44) (end 137.16 91.44) (width 0.25) (layer "B.Cu") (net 2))
 (segment (start 149.86 81.28) (end 139.7 91.44) (width 0.25) (layer "B.Cu") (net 2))
 (segment (start 149.86 93.98) (end 139.7 93.98) (width 0.25) (layer "B.Cu") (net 2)))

